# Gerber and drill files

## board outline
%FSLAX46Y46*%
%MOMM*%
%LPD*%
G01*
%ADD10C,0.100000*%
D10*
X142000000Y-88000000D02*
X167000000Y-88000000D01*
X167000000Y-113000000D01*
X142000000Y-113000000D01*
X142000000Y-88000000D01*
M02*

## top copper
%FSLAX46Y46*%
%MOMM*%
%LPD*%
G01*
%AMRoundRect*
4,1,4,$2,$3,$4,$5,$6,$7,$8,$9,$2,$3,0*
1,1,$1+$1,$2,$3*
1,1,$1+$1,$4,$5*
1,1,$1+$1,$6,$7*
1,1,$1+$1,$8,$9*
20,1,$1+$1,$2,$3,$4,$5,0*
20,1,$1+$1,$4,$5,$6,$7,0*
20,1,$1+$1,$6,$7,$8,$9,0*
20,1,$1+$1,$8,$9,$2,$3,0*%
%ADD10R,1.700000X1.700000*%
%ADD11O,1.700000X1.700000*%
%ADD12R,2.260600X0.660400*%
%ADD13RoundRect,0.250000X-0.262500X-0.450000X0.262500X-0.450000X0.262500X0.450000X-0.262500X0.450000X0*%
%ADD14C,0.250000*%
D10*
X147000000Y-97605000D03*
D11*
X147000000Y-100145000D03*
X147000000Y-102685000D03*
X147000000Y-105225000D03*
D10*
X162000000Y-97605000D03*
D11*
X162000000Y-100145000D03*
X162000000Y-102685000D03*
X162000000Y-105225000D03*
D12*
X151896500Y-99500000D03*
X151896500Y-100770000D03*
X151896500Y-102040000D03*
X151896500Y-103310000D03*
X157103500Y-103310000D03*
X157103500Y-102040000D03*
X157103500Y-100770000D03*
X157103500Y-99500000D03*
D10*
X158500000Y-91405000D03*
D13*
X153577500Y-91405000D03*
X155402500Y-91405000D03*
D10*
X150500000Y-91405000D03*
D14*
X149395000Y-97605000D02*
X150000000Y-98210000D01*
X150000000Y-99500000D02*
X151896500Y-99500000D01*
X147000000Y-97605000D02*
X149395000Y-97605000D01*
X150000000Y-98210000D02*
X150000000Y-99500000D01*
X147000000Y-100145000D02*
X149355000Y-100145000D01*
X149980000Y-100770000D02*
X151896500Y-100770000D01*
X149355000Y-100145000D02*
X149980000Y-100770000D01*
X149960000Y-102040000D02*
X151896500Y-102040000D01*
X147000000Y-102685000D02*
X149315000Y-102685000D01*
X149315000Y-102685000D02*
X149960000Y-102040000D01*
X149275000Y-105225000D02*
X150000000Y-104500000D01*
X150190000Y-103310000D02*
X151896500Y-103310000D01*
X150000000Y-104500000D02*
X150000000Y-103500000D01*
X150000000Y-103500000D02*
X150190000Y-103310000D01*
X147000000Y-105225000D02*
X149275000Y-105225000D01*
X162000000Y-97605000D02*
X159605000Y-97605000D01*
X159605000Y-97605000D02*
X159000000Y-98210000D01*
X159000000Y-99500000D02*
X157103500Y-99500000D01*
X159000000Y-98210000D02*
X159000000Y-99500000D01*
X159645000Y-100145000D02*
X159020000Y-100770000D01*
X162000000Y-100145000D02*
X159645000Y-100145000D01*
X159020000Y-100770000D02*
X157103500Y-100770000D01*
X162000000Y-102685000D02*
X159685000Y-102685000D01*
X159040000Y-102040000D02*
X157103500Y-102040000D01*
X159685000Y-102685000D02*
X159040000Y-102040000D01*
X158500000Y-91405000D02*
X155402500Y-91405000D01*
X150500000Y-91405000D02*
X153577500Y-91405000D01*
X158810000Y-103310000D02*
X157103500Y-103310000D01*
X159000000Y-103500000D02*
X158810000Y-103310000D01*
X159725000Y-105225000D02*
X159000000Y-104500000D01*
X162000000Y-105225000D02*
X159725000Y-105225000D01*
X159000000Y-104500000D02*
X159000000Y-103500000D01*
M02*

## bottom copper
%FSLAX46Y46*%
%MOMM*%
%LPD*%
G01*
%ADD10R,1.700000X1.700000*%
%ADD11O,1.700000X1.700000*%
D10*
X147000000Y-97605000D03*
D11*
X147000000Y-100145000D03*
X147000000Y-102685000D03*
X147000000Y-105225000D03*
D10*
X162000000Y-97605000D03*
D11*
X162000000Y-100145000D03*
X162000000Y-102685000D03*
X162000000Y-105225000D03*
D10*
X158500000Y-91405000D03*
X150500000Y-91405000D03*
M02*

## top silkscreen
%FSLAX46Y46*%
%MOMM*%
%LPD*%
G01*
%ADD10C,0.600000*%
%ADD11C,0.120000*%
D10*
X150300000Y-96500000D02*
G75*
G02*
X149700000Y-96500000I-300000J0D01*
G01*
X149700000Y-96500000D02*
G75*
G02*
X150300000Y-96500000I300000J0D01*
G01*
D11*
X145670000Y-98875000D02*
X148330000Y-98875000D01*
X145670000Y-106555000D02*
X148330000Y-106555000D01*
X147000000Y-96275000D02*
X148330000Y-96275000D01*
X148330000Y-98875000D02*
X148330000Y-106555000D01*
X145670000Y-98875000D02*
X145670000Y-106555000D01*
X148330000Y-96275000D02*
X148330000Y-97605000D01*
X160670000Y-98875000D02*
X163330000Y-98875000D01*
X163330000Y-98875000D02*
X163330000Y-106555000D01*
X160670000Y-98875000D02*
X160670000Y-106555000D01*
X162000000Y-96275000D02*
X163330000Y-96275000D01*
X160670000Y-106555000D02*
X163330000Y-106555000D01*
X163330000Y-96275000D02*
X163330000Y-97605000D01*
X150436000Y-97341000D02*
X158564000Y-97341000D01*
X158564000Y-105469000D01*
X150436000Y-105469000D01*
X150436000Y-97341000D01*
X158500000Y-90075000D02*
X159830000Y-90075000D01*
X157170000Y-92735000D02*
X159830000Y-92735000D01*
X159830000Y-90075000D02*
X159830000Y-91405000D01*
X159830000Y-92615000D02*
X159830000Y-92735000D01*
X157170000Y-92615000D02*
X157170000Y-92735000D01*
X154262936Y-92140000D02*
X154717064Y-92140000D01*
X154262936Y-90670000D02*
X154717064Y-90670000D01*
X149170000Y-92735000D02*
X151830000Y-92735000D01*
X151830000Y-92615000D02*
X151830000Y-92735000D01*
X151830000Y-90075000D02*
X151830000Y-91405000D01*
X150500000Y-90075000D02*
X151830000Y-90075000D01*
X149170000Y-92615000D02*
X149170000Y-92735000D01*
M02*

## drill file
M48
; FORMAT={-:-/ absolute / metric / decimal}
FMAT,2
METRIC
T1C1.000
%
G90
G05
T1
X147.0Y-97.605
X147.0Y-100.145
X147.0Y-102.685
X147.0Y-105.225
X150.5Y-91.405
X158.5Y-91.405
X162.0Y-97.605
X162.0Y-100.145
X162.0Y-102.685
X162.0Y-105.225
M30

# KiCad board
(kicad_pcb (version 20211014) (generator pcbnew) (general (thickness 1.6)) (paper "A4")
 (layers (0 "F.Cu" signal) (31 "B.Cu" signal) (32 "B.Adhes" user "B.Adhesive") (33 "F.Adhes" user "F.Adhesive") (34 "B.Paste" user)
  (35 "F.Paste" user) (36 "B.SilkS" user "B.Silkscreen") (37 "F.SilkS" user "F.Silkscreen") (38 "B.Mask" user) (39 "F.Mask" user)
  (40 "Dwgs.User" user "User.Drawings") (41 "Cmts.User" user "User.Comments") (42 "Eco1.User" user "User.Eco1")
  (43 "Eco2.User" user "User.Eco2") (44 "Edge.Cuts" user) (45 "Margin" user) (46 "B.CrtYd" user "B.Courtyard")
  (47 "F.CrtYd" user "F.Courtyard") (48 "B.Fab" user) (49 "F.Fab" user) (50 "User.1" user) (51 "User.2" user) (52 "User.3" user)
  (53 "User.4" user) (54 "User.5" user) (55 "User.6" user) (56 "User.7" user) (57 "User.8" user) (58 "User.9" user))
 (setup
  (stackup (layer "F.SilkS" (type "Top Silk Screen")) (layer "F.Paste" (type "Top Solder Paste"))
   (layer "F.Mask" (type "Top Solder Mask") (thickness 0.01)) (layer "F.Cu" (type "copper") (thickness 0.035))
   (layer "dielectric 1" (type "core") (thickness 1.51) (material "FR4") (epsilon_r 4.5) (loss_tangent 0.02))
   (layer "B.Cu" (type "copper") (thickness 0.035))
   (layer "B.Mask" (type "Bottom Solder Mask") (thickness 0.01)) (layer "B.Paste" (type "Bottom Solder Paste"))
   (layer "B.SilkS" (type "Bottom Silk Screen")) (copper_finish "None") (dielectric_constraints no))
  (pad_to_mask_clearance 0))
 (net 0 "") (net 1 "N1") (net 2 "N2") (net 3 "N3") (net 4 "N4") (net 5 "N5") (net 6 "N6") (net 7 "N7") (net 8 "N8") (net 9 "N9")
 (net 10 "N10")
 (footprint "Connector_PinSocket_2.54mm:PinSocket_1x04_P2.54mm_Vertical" (layer "F.Cu") (at 147 97.605)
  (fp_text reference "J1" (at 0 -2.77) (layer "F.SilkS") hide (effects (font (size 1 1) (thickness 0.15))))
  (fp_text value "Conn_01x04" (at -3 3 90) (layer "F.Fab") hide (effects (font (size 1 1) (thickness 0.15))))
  (fp_line (start -1.33 1.27) (end 1.33 1.27) (layer "F.SilkS") (width 0.12))
  (fp_line (start -1.33 8.95) (end 1.33 8.95) (layer "F.SilkS") (width 0.12))
  (fp_line (start 0 -1.33) (end 1.33 -1.33) (layer "F.SilkS") (width 0.12))
  (fp_line (start 1.33 1.27) (end 1.33 8.95) (layer "F.SilkS") (width 0.12))
  (fp_line (start -1.33 1.27) (end -1.33 8.95) (layer "F.SilkS") (width 0.12))
  (fp_line (start 1.33 -1.33) (end 1.33 0) (layer "F.SilkS") (width 0.12))
  (pad "1" thru_hole rect (at 0 0) (size 1.7 1.7) (drill 1) (layers *.Cu *.Mask) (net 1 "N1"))
  (pad "2" thru_hole oval (at 0 2.54) (size 1.7 1.7) (drill 1) (layers *.Cu *.Mask) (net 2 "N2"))
  (pad "3" thru_hole oval (at 0 5.08) (size 1.7 1.7) (drill 1) (layers *.Cu *.Mask) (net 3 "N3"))
  (pad "4" thru_hole oval (at 0 7.62) (size 1.7 1.7) (drill 1) (layers *.Cu *.Mask) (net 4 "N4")))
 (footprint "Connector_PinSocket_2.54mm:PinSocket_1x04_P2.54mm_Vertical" (layer "F.Cu") (at 162 97.605)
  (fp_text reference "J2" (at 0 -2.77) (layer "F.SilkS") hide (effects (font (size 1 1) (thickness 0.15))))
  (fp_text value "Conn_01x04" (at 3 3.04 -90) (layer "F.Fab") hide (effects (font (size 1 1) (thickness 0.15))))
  (fp_line (start -1.33 1.27) (end 1.33 1.27) (layer "F.SilkS") (width 0.12))
  (fp_line (start 1.33 1.27) (end 1.33 8.95) (layer "F.SilkS") (width 0.12))
  (fp_line (start -1.33 1.27) (end -1.33 8.95) (layer "F.SilkS") (width 0.12))
  (fp_line (start 0 -1.33) (end 1.33 -1.33) (layer "F.SilkS") (width 0.12))
  (fp_line (start -1.33 8.95) (end 1.33 8.95) (layer "F.SilkS") (width 0.12))
  (fp_line (start 1.33 -1.33) (end 1.33 0) (layer "F.SilkS") (width 0.12))
  (pad "1" thru_hole rect (at 0 0) (size 1.7 1.7) (drill 1) (layers *.Cu *.Mask) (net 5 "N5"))
  (pad "2" thru_hole oval (at 0 2.54) (size 1.7 1.7) (drill 1) (layers *.Cu *.Mask) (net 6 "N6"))
  (pad "3" thru_hole oval (at 0 5.08) (size 1.7 1.7) (drill 1) (layers *.Cu *.Mask) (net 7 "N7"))
  (pad "4" thru_hole oval (at 0 7.62) (size 1.7 1.7) (drill 1) (layers *.Cu *.Mask) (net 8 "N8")))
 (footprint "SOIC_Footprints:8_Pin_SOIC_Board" (layer "F.Cu") (at 154.5 101.405)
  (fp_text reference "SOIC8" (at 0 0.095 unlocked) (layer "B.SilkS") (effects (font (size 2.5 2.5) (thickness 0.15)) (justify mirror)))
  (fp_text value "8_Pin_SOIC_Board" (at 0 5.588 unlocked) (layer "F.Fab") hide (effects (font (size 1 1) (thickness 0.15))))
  (fp_rect (start -4.064 -4.064) (end 4.064 4.064) (layer "F.SilkS") (width 0.12) (fill none))
  (pad "1" smd rect (at -2.6035 -1.905) (size 2.2606 0.6604) (layers "F.Cu" "F.Paste" "F.Mask") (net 1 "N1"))
  (pad "2" smd rect (at -2.6035 -0.635) (size 2.2606 0.6604) (layers "F.Cu" "F.Paste" "F.Mask") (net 2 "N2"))
  (pad "3" smd rect (at -2.6035 0.635) (size 2.2606 0.6604) (layers "F.Cu" "F.Paste" "F.Mask") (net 3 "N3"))
  (pad "4" smd rect (at -2.6035 1.905) (size 2.2606 0.6604) (layers "F.Cu" "F.Paste" "F.Mask") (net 4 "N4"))
  (pad "5" smd rect (at 2.6035 1.905) (size 2.2606 0.6604) (layers "F.Cu" "F.Paste" "F.Mask") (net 8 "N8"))
  (pad "6" smd rect (at 2.6035 0.635) (size 2.2606 0.6604) (layers "F.Cu" "F.Paste" "F.Mask") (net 7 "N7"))
  (pad "7" smd rect (at 2.6035 -0.635) (size 2.2606 0.6604) (layers "F.Cu" "F.Paste" "F.Mask") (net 6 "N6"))
  (pad "8" smd rect (at 2.6035 -1.905) (size 2.2606 0.6604) (layers "F.Cu" "F.Paste" "F.Mask") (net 5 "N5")))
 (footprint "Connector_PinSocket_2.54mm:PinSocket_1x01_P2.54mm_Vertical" (layer "F.Cu") (at 158.5 91.405)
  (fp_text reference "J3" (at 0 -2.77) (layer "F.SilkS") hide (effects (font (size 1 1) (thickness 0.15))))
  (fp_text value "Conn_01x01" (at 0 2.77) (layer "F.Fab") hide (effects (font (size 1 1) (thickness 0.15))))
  (fp_line (start 0 -1.33) (end 1.33 -1.33) (layer "F.SilkS") (width 0.12))
  (fp_line (start -1.33 1.33) (end 1.33 1.33) (layer "F.SilkS") (width 0.12))
  (fp_line (start 1.33 -1.33) (end 1.33 0) (layer "F.SilkS") (width 0.12))
  (fp_line (start 1.33 1.21) (end 1.33 1.33) (layer "F.SilkS") (width 0.12))
  (fp_line (start -1.33 1.21) (end -1.33 1.33) (layer "F.SilkS") (width 0.12))
  (pad "1" thru_hole rect (at 0 0) (size 1.7 1.7) (drill 1) (layers *.Cu *.Mask) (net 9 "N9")))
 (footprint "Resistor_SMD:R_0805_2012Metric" (layer "F.Cu") (at 154.49 91.405)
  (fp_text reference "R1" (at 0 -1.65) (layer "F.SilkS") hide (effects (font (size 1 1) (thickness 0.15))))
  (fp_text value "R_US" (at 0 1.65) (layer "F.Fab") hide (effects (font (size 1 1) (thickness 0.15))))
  (fp_line (start -0.227064 0.735) (end 0.227064 0.735) (layer "F.SilkS") (width 0.12))
  (fp_line (start -0.227064 -0.735) (end 0.227064 -0.735) (layer "F.SilkS") (width 0.12))
  (pad "1" smd roundrect (at -0.9125 0) (size 1.025 1.4) (layers "F.Cu" "F.Paste" "F.Mask") (roundrect_rratio 0.243902) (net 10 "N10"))
  (pad "2" smd roundrect (at 0.9125 0) (size 1.025 1.4) (layers "F.Cu" "F.Paste" "F.Mask") (roundrect_rratio 0.243902) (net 9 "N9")))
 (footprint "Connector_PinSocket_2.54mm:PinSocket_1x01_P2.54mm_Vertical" (layer "F.Cu") (at 150.5 91.405)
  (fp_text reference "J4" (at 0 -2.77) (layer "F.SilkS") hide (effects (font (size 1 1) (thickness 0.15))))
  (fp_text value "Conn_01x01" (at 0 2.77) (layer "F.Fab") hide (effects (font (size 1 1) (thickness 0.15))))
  (fp_line (start -1.33 1.33) (end 1.33 1.33) (layer "F.SilkS") (width 0.12))
  (fp_line (start 1.33 1.21) (end 1.33 1.33) (layer "F.SilkS") (width 0.12))
  (fp_line (start 1.33 -1.33) (end 1.33 0) (layer "F.SilkS") (width 0.12))
  (fp_line (start 0 -1.33) (end 1.33 -1.33) (layer "F.SilkS") (width 0.12))
  (fp_line (start -1.33 1.21) (end -1.33 1.33) (layer "F.SilkS") (width 0.12))
  (pad "1" thru_hole rect (at 0 0) (size 1.7 1.7) (drill 1) (layers *.Cu *.Mask) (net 10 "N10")))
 (gr_circle (center 150 96.5) (end 150.5 96.5) (layer "F.SilkS") (width 0.2) (fill solid))
 (gr_rect (start 142 88) (end 167 113) (layer "Edge.Cuts") (width 0.1) (fill none))
 (segment (start 149.395 97.605) (end 150 98.21) (width 0.25) (layer "F.Cu") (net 1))
 (segment (start 150 99.5) (end 151.8965 99.5) (width 0.25) (layer "F.Cu") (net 1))
 (segment (start 147 97.605) (end 149.395 97.605) (width 0.25) (layer "F.Cu") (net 1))
 (segment (start 150 98.21) (end 150 99.5) (width 0.25) (layer "F.Cu") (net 1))
 (segment (start 147 100.145) (end 149.355 100.145) (width 0.25) (layer "F.Cu") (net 2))
 (segment (start 149.98 100.77) (end 151.8965 100.77) (width 0.25) (layer "F.Cu") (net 2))
 (segment (start 149.355 100.145) (end 149.98 100.77) (width 0.25) (layer "F.Cu") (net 2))
 (segment (start 149.96 102.04) (end 151.8965 102.04) (width 0.25) (layer "F.Cu") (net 3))
 (segment (start 147 102.685) (end 149.315 102.685) (width 0.25) (layer "F.Cu") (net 3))
 (segment (start 149.315 102.685) (end 149.96 102.04) (width 0.25) (layer "F.Cu") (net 3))
 (segment (start 149.275 105.225) (end 150 104.5) (width 0.25) (layer "F.Cu") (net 4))
 (segment (start 150.19 103.31) (end 151.8965 103.31) (width 0.25) (layer "F.Cu") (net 4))
 (segment (start 150 104.5) (end 150 103.5) (width 0.25) (layer "F.Cu") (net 4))
 (segment (start 150 103.5) (end 150.19 103.31) (width 0.25) (layer "F.Cu") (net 4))
 (segment (start 147 105.225) (end 149.275 105.225) (width 0.25) (layer "F.Cu") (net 4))
 (segment (start 162 97.605) (end 159.605 97.605) (width 0.25) (layer "F.Cu") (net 5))
 (segment (start 159.605 97.605) (end 159 98.21) (width 0.25) (layer "F.Cu") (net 5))
 (segment (start 159 99.5) (end 157.1035 99.5) (width 0.25) (layer "F.Cu") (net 5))
 (segment (start 159 98.21) (end 159 99.5) (width 0.25) (layer "F.Cu") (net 5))
 (segment (start 159.645 100.145) (end 159.02 100.77) (width 0.25) (layer "F.Cu") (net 6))
 (segment (start 162 100.145) (end 159.645 100.145) (width 0.25) (layer "F.Cu") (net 6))
 (segment (start 159.02 100.77) (end 157.1035 100.77) (width 0.25) (layer "F.Cu") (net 6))
 (segment (start 162 102.685) (end 159.685 102.685) (width 0.25) (layer "F.Cu") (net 7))
 (segment (start 159.04 102.04) (end 157.1035 102.04) (width 0.25) (layer "F.Cu") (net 7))
 (segment (start 159.685 102.685) (end 159.04 102.04) (width 0.25) (layer "F.Cu") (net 7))
 (segment (start 158.5 91.405) (end 155.4025 91.405) (width 0.25) (layer "F.Cu") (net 9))
 (segment (start 150.5 91.405) (end 153.5775 91.405) (width 0.25) (layer "F.Cu") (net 10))
 (segment (start 158.81 103.31) (end 157.1035 103.31) (width 0.25) (layer "F.Cu") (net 8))
 (segment (start 159 103.5) (end 158.81 103.31) (width 0.25) (layer "F.Cu") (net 8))
 (segment (start 159.725 105.225) (end 159 104.5) (width 0.25) (layer "F.Cu") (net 8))
 (segment (start 162 105.225) (end 159.725 105.225) (width 0.25) (layer "F.Cu") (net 8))
 (segment (start 159 104.5) (end 159 103.5) (width 0.25) (layer "F.Cu") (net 8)))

